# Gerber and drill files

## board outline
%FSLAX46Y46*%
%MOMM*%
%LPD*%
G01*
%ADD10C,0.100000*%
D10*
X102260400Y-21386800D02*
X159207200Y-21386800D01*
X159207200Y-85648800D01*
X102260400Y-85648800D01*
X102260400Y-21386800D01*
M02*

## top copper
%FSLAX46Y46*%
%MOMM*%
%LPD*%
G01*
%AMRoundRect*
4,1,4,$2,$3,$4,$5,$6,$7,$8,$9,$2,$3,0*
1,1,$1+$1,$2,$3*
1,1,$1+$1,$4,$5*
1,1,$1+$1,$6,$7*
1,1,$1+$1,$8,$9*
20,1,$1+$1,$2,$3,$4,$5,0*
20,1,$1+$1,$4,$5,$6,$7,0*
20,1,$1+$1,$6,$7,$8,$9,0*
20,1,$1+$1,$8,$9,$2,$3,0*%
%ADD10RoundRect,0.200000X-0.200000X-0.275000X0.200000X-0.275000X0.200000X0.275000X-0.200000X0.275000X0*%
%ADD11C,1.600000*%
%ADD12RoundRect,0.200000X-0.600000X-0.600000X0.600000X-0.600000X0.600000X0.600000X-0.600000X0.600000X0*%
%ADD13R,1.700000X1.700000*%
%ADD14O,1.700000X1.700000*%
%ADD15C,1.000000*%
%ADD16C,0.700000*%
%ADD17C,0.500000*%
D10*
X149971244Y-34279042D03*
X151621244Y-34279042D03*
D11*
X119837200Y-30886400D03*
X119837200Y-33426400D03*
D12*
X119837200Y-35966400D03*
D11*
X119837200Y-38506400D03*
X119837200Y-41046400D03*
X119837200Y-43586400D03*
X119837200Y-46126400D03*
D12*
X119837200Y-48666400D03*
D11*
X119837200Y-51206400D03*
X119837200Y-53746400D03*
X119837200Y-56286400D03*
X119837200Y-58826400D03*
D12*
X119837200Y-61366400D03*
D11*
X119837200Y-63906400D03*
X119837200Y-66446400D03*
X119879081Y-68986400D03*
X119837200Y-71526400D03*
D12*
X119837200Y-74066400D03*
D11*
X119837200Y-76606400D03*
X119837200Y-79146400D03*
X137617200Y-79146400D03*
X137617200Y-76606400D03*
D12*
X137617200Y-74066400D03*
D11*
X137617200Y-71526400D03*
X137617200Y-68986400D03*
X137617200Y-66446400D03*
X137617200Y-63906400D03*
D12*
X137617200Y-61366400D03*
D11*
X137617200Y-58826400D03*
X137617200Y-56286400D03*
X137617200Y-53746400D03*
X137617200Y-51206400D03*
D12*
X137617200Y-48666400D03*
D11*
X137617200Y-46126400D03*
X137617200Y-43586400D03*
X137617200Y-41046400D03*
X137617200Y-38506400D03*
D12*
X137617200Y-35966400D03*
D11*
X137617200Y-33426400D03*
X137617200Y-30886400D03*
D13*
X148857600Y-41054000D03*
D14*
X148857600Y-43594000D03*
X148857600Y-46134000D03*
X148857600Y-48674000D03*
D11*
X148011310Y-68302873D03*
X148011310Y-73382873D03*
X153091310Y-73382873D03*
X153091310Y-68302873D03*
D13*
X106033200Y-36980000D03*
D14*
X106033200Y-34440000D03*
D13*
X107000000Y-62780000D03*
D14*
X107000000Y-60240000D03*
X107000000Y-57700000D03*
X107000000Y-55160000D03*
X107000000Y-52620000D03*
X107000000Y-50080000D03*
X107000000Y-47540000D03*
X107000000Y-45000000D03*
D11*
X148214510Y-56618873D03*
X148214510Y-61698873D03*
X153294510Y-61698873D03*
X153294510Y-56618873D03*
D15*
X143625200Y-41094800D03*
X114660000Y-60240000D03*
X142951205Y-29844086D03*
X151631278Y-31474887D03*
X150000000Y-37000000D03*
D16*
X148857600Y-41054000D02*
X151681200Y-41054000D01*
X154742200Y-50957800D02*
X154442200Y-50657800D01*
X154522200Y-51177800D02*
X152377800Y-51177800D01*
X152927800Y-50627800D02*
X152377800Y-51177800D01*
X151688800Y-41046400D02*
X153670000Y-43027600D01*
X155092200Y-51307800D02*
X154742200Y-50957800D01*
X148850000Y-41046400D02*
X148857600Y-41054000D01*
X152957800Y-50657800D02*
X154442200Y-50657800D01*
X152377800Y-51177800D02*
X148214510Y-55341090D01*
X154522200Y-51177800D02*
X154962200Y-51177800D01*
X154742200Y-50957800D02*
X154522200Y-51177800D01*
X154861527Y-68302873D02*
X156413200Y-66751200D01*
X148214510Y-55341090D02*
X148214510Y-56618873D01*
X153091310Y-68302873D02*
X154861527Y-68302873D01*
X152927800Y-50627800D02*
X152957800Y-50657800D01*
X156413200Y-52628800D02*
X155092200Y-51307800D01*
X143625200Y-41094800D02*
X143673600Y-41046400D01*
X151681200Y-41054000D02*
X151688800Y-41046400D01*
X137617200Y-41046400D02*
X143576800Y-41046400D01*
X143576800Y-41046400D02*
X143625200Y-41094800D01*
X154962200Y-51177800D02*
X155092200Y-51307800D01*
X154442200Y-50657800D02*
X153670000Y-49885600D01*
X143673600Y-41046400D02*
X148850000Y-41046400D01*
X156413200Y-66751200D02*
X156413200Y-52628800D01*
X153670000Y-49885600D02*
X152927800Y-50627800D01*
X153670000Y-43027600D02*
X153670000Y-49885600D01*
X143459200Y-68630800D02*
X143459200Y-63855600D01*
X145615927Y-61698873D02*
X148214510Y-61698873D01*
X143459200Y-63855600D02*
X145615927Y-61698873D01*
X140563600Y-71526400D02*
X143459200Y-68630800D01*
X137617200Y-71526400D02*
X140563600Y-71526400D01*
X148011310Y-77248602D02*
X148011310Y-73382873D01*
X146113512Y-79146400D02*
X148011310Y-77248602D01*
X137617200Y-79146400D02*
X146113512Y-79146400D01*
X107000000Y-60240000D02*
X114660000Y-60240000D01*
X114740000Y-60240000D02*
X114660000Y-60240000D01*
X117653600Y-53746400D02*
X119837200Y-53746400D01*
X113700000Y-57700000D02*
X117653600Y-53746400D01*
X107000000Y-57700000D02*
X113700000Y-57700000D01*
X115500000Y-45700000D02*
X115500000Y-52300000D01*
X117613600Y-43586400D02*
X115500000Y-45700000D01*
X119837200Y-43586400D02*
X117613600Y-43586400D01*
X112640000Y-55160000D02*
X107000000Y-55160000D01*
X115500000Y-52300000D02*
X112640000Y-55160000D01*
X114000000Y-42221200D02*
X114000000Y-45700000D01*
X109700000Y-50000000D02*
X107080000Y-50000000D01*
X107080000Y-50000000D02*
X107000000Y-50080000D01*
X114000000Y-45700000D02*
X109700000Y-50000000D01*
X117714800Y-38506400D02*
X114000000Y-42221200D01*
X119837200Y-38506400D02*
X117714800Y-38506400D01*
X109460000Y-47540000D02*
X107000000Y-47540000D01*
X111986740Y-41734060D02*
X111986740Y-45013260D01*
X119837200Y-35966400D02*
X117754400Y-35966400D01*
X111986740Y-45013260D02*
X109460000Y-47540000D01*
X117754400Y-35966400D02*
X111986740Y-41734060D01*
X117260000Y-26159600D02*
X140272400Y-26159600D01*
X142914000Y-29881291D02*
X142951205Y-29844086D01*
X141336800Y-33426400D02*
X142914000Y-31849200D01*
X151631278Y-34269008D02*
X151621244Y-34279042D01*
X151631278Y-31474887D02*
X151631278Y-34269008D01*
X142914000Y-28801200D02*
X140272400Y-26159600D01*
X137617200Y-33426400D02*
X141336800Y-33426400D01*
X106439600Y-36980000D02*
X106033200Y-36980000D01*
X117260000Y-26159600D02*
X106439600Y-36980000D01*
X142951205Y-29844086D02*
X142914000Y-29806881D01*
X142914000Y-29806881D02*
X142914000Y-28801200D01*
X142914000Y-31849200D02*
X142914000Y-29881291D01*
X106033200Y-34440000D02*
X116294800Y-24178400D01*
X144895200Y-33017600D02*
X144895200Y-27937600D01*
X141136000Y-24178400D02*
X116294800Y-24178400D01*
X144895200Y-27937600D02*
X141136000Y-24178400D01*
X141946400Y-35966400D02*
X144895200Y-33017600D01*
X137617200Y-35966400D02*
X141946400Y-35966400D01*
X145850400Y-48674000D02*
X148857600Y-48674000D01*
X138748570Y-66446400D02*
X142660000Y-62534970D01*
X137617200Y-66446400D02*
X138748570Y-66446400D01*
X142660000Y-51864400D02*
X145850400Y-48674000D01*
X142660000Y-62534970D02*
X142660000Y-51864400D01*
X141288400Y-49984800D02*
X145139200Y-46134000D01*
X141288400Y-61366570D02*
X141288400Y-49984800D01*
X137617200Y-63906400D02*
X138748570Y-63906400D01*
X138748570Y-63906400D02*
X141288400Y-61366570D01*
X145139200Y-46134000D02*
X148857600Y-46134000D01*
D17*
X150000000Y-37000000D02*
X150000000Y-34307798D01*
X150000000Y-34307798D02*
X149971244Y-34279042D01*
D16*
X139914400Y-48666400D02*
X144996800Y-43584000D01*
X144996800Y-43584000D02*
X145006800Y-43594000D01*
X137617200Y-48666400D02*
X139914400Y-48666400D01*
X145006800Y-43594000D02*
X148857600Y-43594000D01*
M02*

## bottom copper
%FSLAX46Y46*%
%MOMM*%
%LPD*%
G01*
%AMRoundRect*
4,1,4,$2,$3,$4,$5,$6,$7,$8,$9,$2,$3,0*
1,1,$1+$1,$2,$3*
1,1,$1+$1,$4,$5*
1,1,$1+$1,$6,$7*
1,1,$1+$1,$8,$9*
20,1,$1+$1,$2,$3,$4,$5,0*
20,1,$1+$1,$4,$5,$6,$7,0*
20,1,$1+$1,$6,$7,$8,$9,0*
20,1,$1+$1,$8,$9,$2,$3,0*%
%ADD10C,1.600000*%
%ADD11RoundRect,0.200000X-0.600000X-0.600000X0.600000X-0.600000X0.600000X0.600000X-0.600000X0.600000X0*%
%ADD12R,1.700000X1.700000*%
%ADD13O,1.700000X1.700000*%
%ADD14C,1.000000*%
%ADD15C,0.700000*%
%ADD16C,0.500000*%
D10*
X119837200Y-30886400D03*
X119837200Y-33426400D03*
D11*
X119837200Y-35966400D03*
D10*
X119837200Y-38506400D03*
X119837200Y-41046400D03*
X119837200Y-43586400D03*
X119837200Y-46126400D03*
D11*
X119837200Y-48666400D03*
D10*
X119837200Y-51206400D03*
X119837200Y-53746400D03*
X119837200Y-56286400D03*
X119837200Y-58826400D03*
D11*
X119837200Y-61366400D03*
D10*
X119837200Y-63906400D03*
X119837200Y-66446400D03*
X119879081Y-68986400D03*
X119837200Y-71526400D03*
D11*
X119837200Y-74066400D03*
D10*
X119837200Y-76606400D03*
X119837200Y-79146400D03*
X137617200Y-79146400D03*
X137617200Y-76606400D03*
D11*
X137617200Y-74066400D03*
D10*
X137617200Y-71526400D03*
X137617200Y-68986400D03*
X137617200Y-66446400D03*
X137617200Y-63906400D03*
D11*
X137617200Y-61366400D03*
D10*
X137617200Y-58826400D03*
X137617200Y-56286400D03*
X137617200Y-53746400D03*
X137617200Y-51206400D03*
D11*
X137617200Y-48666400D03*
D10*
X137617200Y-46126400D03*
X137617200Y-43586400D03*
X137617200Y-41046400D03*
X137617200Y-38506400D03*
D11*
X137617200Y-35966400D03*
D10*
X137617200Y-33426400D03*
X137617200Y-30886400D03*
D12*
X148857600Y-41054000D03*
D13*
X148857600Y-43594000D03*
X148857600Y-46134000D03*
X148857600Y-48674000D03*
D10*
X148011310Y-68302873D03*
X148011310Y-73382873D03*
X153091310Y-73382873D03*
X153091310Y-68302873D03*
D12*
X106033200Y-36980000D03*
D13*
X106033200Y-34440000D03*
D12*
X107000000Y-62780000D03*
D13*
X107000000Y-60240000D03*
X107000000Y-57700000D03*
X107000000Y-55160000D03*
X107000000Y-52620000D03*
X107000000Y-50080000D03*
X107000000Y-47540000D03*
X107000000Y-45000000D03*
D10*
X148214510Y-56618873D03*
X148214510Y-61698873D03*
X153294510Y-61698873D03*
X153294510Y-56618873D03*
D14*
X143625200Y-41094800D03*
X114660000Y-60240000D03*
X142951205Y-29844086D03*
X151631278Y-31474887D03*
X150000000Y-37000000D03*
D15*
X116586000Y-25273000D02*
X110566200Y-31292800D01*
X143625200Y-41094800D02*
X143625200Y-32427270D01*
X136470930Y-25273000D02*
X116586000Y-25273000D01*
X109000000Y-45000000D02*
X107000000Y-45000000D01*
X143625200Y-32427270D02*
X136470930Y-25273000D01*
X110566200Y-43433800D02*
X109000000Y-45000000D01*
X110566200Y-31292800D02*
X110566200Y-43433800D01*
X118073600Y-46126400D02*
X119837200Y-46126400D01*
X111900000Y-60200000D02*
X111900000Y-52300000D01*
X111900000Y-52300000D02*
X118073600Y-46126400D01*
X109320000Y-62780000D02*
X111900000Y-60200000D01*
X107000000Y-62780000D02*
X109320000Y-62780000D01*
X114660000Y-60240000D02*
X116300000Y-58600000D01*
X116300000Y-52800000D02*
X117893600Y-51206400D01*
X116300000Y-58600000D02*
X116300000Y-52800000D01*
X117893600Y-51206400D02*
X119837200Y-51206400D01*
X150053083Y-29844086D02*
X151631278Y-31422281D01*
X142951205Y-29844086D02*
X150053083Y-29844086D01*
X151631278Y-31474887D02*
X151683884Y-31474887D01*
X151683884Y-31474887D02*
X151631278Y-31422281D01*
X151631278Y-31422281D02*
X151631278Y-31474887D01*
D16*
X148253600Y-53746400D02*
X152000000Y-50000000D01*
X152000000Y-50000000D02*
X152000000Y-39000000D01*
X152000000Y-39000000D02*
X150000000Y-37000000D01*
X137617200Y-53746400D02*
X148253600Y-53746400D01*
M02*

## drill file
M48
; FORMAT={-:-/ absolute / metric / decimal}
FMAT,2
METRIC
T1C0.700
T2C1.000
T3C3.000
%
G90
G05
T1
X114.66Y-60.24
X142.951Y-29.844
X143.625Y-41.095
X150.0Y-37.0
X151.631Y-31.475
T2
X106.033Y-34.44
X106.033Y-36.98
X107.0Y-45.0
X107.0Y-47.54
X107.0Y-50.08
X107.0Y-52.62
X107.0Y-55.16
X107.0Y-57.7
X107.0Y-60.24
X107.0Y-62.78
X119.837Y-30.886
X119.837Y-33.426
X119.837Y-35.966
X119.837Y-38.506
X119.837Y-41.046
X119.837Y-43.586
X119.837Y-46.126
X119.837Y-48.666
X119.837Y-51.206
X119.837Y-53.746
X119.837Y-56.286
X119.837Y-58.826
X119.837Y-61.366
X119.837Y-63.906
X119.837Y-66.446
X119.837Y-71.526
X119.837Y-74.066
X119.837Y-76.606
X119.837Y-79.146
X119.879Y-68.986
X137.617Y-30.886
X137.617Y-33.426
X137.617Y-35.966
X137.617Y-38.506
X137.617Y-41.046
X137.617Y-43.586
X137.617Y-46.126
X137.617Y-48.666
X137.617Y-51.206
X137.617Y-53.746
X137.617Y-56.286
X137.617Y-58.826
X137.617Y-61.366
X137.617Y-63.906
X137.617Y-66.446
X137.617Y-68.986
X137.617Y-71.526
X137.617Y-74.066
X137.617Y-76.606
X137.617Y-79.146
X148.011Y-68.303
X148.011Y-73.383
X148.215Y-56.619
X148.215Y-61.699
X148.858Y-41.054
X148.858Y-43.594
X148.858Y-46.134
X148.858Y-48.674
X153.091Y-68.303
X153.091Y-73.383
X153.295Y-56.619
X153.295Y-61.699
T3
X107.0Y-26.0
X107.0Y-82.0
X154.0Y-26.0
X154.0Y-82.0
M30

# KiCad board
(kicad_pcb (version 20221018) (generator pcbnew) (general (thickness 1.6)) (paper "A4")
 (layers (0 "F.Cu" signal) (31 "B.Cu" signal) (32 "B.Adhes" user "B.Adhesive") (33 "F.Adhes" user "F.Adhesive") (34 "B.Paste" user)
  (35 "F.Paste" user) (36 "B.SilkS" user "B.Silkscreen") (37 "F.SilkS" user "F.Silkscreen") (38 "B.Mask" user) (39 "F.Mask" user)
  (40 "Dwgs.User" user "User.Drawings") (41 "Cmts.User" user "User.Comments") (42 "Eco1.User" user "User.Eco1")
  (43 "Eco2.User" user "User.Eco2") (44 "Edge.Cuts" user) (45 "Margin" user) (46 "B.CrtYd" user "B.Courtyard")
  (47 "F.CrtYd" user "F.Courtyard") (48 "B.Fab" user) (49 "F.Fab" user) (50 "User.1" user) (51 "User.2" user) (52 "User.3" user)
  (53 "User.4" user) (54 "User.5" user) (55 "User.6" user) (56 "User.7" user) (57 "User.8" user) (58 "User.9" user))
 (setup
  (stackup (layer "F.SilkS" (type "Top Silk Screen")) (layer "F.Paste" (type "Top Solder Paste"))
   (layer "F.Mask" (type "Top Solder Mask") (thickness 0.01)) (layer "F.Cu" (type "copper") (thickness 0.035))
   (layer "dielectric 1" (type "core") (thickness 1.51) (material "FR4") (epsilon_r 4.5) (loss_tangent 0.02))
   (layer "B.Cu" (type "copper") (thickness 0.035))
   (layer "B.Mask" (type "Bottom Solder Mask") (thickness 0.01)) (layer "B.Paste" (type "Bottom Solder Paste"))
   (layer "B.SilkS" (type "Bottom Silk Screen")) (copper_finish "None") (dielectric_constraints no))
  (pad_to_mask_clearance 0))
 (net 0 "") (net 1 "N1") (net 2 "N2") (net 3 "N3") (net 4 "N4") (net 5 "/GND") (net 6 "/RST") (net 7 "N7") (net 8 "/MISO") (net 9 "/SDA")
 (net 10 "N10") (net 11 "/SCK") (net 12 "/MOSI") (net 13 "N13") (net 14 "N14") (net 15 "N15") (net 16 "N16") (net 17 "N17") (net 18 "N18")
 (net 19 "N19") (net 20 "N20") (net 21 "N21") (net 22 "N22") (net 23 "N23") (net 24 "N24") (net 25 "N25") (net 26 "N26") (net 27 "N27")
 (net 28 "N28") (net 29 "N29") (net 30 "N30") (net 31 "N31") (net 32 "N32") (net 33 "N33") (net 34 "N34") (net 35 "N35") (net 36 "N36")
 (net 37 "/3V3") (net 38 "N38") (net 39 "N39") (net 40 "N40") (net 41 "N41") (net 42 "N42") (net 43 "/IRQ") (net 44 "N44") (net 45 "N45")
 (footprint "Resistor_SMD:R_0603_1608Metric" (layer "F.Cu") (at 150.796244 34.279042)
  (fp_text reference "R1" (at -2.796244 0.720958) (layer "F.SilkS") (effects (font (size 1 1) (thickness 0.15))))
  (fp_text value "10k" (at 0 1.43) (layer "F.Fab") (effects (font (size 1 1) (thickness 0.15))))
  (pad "1" smd roundrect (at -0.825 0) (size 0.8 0.95) (layers "F.Cu" "F.Paste" "F.Mask") (roundrect_rratio 0.25) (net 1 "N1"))
  (pad "2" smd roundrect (at 0.825 0) (size 0.8 0.95) (layers "F.Cu" "F.Paste" "F.Mask") (roundrect_rratio 0.25) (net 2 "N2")))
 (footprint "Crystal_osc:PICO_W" (layer "F.Cu") (at 128.7272 55.0164)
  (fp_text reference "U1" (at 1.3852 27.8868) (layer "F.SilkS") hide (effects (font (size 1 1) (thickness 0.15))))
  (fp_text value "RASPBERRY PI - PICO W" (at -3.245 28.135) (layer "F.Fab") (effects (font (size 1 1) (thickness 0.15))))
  (pad "1" thru_hole circle (at -8.89 -24.13) (size 1.6 1.6) (drill 1) (layers "*.Cu" "*.Mask") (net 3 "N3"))
  (pad "2" thru_hole circle (at -8.89 -21.59) (size 1.6 1.6) (drill 1) (layers "*.Cu" "*.Mask") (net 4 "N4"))
  (pad "3" thru_hole roundrect (at -8.89 -19.05) (size 1.6 1.6) (drill 1) (layers "*.Cu" "*.Mask") (roundrect_rratio 0.125) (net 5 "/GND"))
  (pad "4" thru_hole circle (at -8.89 -16.51) (size 1.6 1.6) (drill 1) (layers "*.Cu" "*.Mask") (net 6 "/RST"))
  (pad "5" thru_hole circle (at -8.89 -13.97) (size 1.6 1.6) (drill 1) (layers "*.Cu" "*.Mask") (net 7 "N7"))
  (pad "6" thru_hole circle (at -8.89 -11.43) (size 1.6 1.6) (drill 1) (layers "*.Cu" "*.Mask") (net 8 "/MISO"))
  (pad "7" thru_hole circle (at -8.89 -8.89) (size 1.6 1.6) (drill 1) (layers "*.Cu" "*.Mask") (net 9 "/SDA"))
  (pad "8" thru_hole roundrect (at -8.89 -6.35) (size 1.6 1.6) (drill 1) (layers "*.Cu" "*.Mask") (roundrect_rratio 0.125) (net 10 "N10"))
  (pad "9" thru_hole circle (at -8.89 -3.81) (size 1.6 1.6) (drill 1) (layers "*.Cu" "*.Mask") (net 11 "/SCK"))
  (pad "10" thru_hole circle (at -8.89 -1.27) (size 1.6 1.6) (drill 1) (layers "*.Cu" "*.Mask") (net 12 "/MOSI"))
  (pad "11" thru_hole circle (at -8.89 1.27) (size 1.6 1.6) (drill 1) (layers "*.Cu" "*.Mask") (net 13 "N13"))
  (pad "12" thru_hole circle (at -8.89 3.81) (size 1.6 1.6) (drill 1) (layers "*.Cu" "*.Mask") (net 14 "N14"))
  (pad "13" thru_hole roundrect (at -8.89 6.35) (size 1.6 1.6) (drill 1) (layers "*.Cu" "*.Mask") (roundrect_rratio 0.125) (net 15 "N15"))
  (pad "14" thru_hole circle (at -8.89 8.89) (size 1.6 1.6) (drill 1) (layers "*.Cu" "*.Mask") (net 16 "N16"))
  (pad "15" thru_hole circle (at -8.89 11.43) (size 1.6 1.6) (drill 1) (layers "*.Cu" "*.Mask") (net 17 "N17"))
  (pad "16" thru_hole circle (at -8.848119 13.97) (size 1.6 1.6) (drill 1) (layers "*.Cu" "*.Mask") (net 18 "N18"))
  (pad "17" thru_hole circle (at -8.89 16.51) (size 1.6 1.6) (drill 1) (layers "*.Cu" "*.Mask") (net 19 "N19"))
  (pad "18" thru_hole roundrect (at -8.89 19.05) (size 1.6 1.6) (drill 1) (layers "*.Cu" "*.Mask") (roundrect_rratio 0.125) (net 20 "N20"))
  (pad "19" thru_hole circle (at -8.89 21.59) (size 1.6 1.6) (drill 1) (layers "*.Cu" "*.Mask") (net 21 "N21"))
  (pad "20" thru_hole circle (at -8.89 24.13) (size 1.6 1.6) (drill 1) (layers "*.Cu" "*.Mask") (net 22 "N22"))
  (pad "21" thru_hole circle (at 8.89 24.13) (size 1.6 1.6) (drill 1) (layers "*.Cu" "*.Mask") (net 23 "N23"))
  (pad "22" thru_hole circle (at 8.89 21.59) (size 1.6 1.6) (drill 1) (layers "*.Cu" "*.Mask") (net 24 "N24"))
  (pad "23" thru_hole roundrect (at 8.89 19.05) (size 1.6 1.6) (drill 1) (layers "*.Cu" "*.Mask") (roundrect_rratio 0.125) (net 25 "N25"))
  (pad "24" thru_hole circle (at 8.89 16.51) (size 1.6 1.6) (drill 1) (layers "*.Cu" "*.Mask") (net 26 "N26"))
  (pad "25" thru_hole circle (at 8.89 13.97) (size 1.6 1.6) (drill 1) (layers "*.Cu" "*.Mask") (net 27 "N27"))
  (pad "26" thru_hole circle (at 8.89 11.43) (size 1.6 1.6) (drill 1) (layers "*.Cu" "*.Mask") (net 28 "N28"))
  (pad "27" thru_hole circle (at 8.89 8.89) (size 1.6 1.6) (drill 1) (layers "*.Cu" "*.Mask") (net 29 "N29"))
  (pad "28" thru_hole roundrect (at 8.89 6.35) (size 1.6 1.6) (drill 1) (layers "*.Cu" "*.Mask") (roundrect_rratio 0.125) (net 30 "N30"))
  (pad "29" thru_hole circle (at 8.89 3.81) (size 1.6 1.6) (drill 1) (layers "*.Cu" "*.Mask") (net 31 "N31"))
  (pad "30" thru_hole circle (at 8.89 1.27) (size 1.6 1.6) (drill 1) (layers "*.Cu" "*.Mask") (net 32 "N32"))
  (pad "31" thru_hole circle (at 8.89 -1.27) (size 1.6 1.6) (drill 1) (layers "*.Cu" "*.Mask") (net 1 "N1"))
  (pad "32" thru_hole circle (at 8.89 -3.81) (size 1.6 1.6) (drill 1) (layers "*.Cu" "*.Mask") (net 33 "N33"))
  (pad "33" thru_hole roundrect (at 8.89 -6.35) (size 1.6 1.6) (drill 1) (layers "*.Cu" "*.Mask") (roundrect_rratio 0.125) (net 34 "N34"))
  (pad "34" thru_hole circle (at 8.89 -8.89) (size 1.6 1.6) (drill 1) (layers "*.Cu" "*.Mask") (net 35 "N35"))
  (pad "35" thru_hole circle (at 8.89 -11.43) (size 1.6 1.6) (drill 1) (layers "*.Cu" "*.Mask") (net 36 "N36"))
  (pad "36" thru_hole circle (at 8.89 -13.97) (size 1.6 1.6) (drill 1) (layers "*.Cu" "*.Mask") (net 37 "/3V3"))
  (pad "37" thru_hole circle (at 8.89 -16.51) (size 1.6 1.6) (drill 1) (layers "*.Cu" "*.Mask") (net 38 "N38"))
  (pad "38" thru_hole roundrect (at 8.89 -19.05) (size 1.6 1.6) (drill 1) (layers "*.Cu" "*.Mask") (roundrect_rratio 0.125) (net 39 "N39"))
  (pad "39" thru_hole circle (at 8.89 -21.59) (size 1.6 1.6) (drill 1) (layers "*.Cu" "*.Mask") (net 2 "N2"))
  (pad "40" thru_hole circle (at 8.89 -24.13) (size 1.6 1.6) (drill 1) (layers "*.Cu" "*.Mask") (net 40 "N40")))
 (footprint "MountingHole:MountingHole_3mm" (layer "F.Cu") (at 154 82)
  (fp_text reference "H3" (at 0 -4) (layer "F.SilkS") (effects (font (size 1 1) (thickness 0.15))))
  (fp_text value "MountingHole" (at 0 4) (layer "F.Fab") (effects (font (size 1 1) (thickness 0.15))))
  (pad "" np_thru_hole circle (at 0 0) (size 3 3) (drill 3) (layers "*.Cu" "*.Mask")))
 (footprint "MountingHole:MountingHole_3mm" (layer "F.Cu") (at 154 26)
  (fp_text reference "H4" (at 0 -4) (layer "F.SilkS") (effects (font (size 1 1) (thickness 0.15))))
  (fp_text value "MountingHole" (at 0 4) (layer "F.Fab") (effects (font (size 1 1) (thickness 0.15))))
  (pad "" np_thru_hole circle (at 0 0) (size 3 3) (drill 3) (layers "*.Cu" "*.Mask")))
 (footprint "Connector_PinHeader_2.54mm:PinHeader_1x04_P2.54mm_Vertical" (layer "F.Cu") (at 148.8576 41.054)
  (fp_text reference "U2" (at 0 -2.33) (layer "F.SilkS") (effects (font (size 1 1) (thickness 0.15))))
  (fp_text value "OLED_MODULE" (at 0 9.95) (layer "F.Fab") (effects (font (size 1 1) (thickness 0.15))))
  (pad "1" thru_hole rect (at 0 0) (size 1.7 1.7) (drill 1) (layers "*.Cu" "*.Mask") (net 37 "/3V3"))
  (pad "2" thru_hole oval (at 0 2.54) (size 1.7 1.7) (drill 1) (layers "*.Cu" "*.Mask") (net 34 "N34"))
  (pad "3" thru_hole oval (at 0 5.08) (size 1.7 1.7) (drill 1) (layers "*.Cu" "*.Mask") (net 29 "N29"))
  (pad "4" thru_hole oval (at 0 7.62) (size 1.7 1.7) (drill 1) (layers "*.Cu" "*.Mask") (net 28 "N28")))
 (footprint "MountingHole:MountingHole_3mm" (layer "F.Cu") (at 107 82)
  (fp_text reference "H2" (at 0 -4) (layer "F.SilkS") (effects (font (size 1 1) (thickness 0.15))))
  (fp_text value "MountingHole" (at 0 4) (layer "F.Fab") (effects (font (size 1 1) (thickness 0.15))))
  (pad "" np_thru_hole circle (at 0 0) (size 3 3) (drill 3) (layers "*.Cu" "*.Mask")))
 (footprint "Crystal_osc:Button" (layer "F.Cu") (at 150.55131 60.682873)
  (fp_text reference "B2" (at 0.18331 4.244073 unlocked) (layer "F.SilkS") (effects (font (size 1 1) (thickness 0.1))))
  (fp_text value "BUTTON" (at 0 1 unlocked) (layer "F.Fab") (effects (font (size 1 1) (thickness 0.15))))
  (pad "1" thru_hole circle (at -2.54 7.62) (size 1.6 1.6) (drill 1) (layers "*.Cu" "*.Mask") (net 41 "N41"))
  (pad "2" thru_hole circle (at -2.54 12.7) (size 1.6 1.6) (drill 1) (layers "*.Cu" "*.Mask") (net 23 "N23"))
  (pad "3" thru_hole circle (at 2.54 12.7 180) (size 1.6 1.6) (drill 1) (layers "*.Cu" "*.Mask") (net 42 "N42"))
  (pad "4" thru_hole circle (at 2.54 7.62 90) (size 1.6 1.6) (drill 1) (layers "*.Cu" "*.Mask") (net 37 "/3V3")))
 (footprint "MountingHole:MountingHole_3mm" (layer "F.Cu") (at 107 26)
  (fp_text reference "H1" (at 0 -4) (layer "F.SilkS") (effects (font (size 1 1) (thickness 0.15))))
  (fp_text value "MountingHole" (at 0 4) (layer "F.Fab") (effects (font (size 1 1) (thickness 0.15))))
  (pad "" np_thru_hole circle (at 0 0) (size 3 3) (drill 3) (layers "*.Cu" "*.Mask")))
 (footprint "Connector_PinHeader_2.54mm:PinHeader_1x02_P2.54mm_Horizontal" (layer "F.Cu") (at 106.0332 36.98 180)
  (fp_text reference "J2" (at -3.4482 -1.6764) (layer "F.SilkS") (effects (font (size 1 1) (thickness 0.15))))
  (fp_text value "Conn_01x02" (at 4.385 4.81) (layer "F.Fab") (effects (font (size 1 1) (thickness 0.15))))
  (pad "1" thru_hole rect (at 0 0 180) (size 1.7 1.7) (drill 1) (layers "*.Cu" "*.Mask") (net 2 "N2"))
  (pad "2" thru_hole oval (at 0 2.54 180) (size 1.7 1.7) (drill 1) (layers "*.Cu" "*.Mask") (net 39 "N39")))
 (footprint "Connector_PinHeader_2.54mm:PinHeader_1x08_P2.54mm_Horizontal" (layer "F.Cu") (at 107 62.78 180)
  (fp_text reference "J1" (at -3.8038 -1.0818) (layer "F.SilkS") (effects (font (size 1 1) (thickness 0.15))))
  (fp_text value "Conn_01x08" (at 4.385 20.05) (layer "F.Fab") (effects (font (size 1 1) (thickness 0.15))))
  (pad "1" thru_hole rect (at 0 0 180) (size 1.7 1.7) (drill 1) (layers "*.Cu" "*.Mask") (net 9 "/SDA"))
  (pad "2" thru_hole oval (at 0 2.54 180) (size 1.7 1.7) (drill 1) (layers "*.Cu" "*.Mask") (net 11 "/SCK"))
  (pad "3" thru_hole oval (at 0 5.08 180) (size 1.7 1.7) (drill 1) (layers "*.Cu" "*.Mask") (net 12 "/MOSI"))
  (pad "4" thru_hole oval (at 0 7.62 180) (size 1.7 1.7) (drill 1) (layers "*.Cu" "*.Mask") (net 8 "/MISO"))
  (pad "5" thru_hole oval (at 0 10.16 180) (size 1.7 1.7) (drill 1) (layers "*.Cu" "*.Mask") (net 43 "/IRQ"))
  (pad "6" thru_hole oval (at 0 12.7 180) (size 1.7 1.7) (drill 1) (layers "*.Cu" "*.Mask") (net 6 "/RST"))
  (pad "7" thru_hole oval (at 0 15.24 180) (size 1.7 1.7) (drill 1) (layers "*.Cu" "*.Mask") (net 5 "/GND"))
  (pad "8" thru_hole oval (at 0 17.78 180) (size 1.7 1.7) (drill 1) (layers "*.Cu" "*.Mask") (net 37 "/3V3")))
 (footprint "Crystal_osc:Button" (layer "F.Cu") (at 150.75451 48.998873)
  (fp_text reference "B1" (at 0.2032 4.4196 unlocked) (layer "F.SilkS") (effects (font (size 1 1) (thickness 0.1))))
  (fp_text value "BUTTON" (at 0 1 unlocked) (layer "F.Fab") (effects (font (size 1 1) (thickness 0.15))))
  (pad "1" thru_hole circle (at -2.54 7.62) (size 1.6 1.6) (drill 1) (layers "*.Cu" "*.Mask") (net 37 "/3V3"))
  (pad "2" thru_hole circle (at -2.54 12.7) (size 1.6 1.6) (drill 1) (layers "*.Cu" "*.Mask") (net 26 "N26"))
  (pad "3" thru_hole circle (at 2.54 12.7 180) (size 1.6 1.6) (drill 1) (layers "*.Cu" "*.Mask") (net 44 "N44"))
  (pad "4" thru_hole circle (at 2.54 7.62 90) (size 1.6 1.6) (drill 1) (layers "*.Cu" "*.Mask") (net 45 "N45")))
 (gr_rect (start 102.2604 21.3868) (end 159.2072 85.6488) (stroke (width 0.1) (type default)) (fill none) (layer "Edge.Cuts"))
 (segment (start 148.8576 41.054) (end 151.6812 41.054) (width 0.7) (layer "F.Cu") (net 37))
 (segment (start 154.7422 50.9578) (end 154.4422 50.6578) (width 0.7) (layer "F.Cu") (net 37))
 (segment (start 154.5222 51.1778) (end 152.3778 51.1778) (width 0.7) (layer "F.Cu") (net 37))
 (segment (start 152.9278 50.6278) (end 152.3778 51.1778) (width 0.7) (layer "F.Cu") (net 37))
 (segment (start 151.6888 41.0464) (end 153.67 43.0276) (width 0.7) (layer "F.Cu") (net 37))
 (segment (start 155.0922 51.3078) (end 154.7422 50.9578) (width 0.7) (layer "F.Cu") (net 37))
 (segment (start 148.85 41.0464) (end 148.8576 41.054) (width 0.7) (layer "F.Cu") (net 37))
 (segment (start 152.9578 50.6578) (end 154.4422 50.6578) (width 0.7) (layer "F.Cu") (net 37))
 (segment (start 152.3778 51.1778) (end 148.21451 55.34109) (width 0.7) (layer "F.Cu") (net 37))
 (segment (start 154.5222 51.1778) (end 154.9622 51.1778) (width 0.7) (layer "F.Cu") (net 37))
 (segment (start 154.7422 50.9578) (end 154.5222 51.1778) (width 0.7) (layer "F.Cu") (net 37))
 (segment (start 154.861527 68.302873) (end 156.4132 66.7512) (width 0.7) (layer "F.Cu") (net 37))
 (segment (start 148.21451 55.34109) (end 148.21451 56.618873) (width 0.7) (layer "F.Cu") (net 37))
 (segment (start 153.09131 68.302873) (end 154.861527 68.302873) (width 0.7) (layer "F.Cu") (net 37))
 (segment (start 152.9278 50.6278) (end 152.9578 50.6578) (width 0.7) (layer "F.Cu") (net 37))
 (segment (start 156.4132 52.6288) (end 155.0922 51.3078) (width 0.7) (layer "F.Cu") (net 37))
 (segment (start 143.6252 41.0948) (end 143.6736 41.0464) (width 0.7) (layer "F.Cu") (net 37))
 (segment (start 151.6812 41.054) (end 151.6888 41.0464) (width 0.7) (layer "F.Cu") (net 37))
 (segment (start 137.6172 41.0464) (end 143.5768 41.0464) (width 0.7) (layer "F.Cu") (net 37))
 (segment (start 143.5768 41.0464) (end 143.6252 41.0948) (width 0.7) (layer "F.Cu") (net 37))
 (segment (start 154.9622 51.1778) (end 155.0922 51.3078) (width 0.7) (layer "F.Cu") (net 37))
 (segment (start 154.4422 50.6578) (end 153.67 49.8856) (width 0.7) (layer "F.Cu") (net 37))
 (segment (start 143.6736 41.0464) (end 148.85 41.0464) (width 0.7) (layer "F.Cu") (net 37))
 (segment (start 156.4132 66.7512) (end 156.4132 52.6288) (width 0.7) (layer "F.Cu") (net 37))
 (segment (start 153.67 49.8856) (end 152.9278 50.6278) (width 0.7) (layer "F.Cu") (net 37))
 (segment (start 153.67 43.0276) (end 153.67 49.8856) (width 0.7) (layer "F.Cu") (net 37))
 (via (at 143.6252 41.0948) (size 1) (drill 0.7) (layers "F.Cu" "B.Cu") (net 37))
 (segment (start 116.586 25.273) (end 110.5662 31.2928) (width 0.7) (layer "B.Cu") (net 37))
 (segment (start 143.6252 41.0948) (end 143.6252 32.42727) (width 0.7) (layer "B.Cu") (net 37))
 (segment (start 136.47093 25.273) (end 116.586 25.273) (width 0.7) (layer "B.Cu") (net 37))
 (segment (start 109 45) (end 107 45) (width 0.7) (layer "B.Cu") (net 37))
 (segment (start 143.6252 32.42727) (end 136.47093 25.273) (width 0.7) (layer "B.Cu") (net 37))
 (segment (start 110.5662 43.4338) (end 109 45) (width 0.7) (layer "B.Cu") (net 37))
 (segment (start 110.5662 31.2928) (end 110.5662 43.4338) (width 0.7) (layer "B.Cu") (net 37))
 (segment (start 143.4592 68.6308) (end 143.4592 63.8556) (width 0.7) (layer "F.Cu") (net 26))
 (segment (start 145.615927 61.698873) (end 148.21451 61.698873) (width 0.7) (layer "F.Cu") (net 26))
 (segment (start 143.4592 63.8556) (end 145.615927 61.698873) (width 0.7) (layer "F.Cu") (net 26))
 (segment (start 140.5636 71.5264) (end 143.4592 68.6308) (width 0.7) (layer "F.Cu") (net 26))
 (segment (start 137.6172 71.5264) (end 140.5636 71.5264) (width 0.7) (layer "F.Cu") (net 26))
 (segment (start 148.01131 77.248602) (end 148.01131 73.382873) (width 0.7) (layer "F.Cu") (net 23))
 (segment (start 146.113512 79.1464) (end 148.01131 77.248602) (width 0.7) (layer "F.Cu") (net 23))
 (segment (start 137.6172 79.1464) (end 146.113512 79.1464) (width 0.7) (layer "F.Cu") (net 23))
 (segment (start 118.0736 46.1264) (end 119.8372 46.1264) (width 0.7) (layer "B.Cu") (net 9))
 (segment (start 111.9 60.2) (end 111.9 52.3) (width 0.7) (layer "B.Cu") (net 9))
 (segment (start 111.9 52.3) (end 118.0736 46.1264) (width 0.7) (layer "B.Cu") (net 9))
 (segment (start 109.32 62.78) (end 111.9 60.2) (width 0.7) (layer "B.Cu") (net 9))
 (segment (start 107 62.78) (end 109.32 62.78) (width 0.7) (layer "B.Cu") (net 9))
 (segment (start 107 60.24) (end 114.66 60.24) (width 0.7) (layer "F.Cu") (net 11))
 (segment (start 114.74 60.24) (end 114.66 60.24) (width 0.7) (layer "F.Cu") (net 11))
 (via (at 114.66 60.24) (size 1) (drill 0.7) (layers "F.Cu" "B.Cu") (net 11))
 (segment (start 114.66 60.24) (end 116.3 58.6) (width 0.7) (layer "B.Cu") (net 11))
 (segment (start 116.3 52.8) (end 117.8936 51.2064) (width 0.7) (layer "B.Cu") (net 11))
 (segment (start 116.3 58.6) (end 116.3 52.8) (width 0.7) (layer "B.Cu") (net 11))
 (segment (start 117.8936 51.2064) (end 119.8372 51.2064) (width 0.7) (layer "B.Cu") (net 11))
 (segment (start 117.6536 53.7464) (end 119.8372 53.7464) (width 0.7) (layer "F.Cu") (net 12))
 (segment (start 113.7 57.7) (end 117.6536 53.7464) (width 0.7) (layer "F.Cu") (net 12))
 (segment (start 107 57.7) (end 113.7 57.7) (width 0.7) (layer "F.Cu") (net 12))
 (segment (start 115.5 45.7) (end 115.5 52.3) (width 0.7) (layer "F.Cu") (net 8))
 (segment (start 117.6136 43.5864) (end 115.5 45.7) (width 0.7) (layer "F.Cu") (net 8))
 (segment (start 119.8372 43.5864) (end 117.6136 43.5864) (width 0.7) (layer "F.Cu") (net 8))
 (segment (start 112.64 55.16) (end 107 55.16) (width 0.7) (layer "F.Cu") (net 8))
 (segment (start 115.5 52.3) (end 112.64 55.16) (width 0.7) (layer "F.Cu") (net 8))
 (segment (start 114 42.2212) (end 114 45.7) (width 0.7) (layer "F.Cu") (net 6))
 (segment (start 109.7 50) (end 107.08 50) (width 0.7) (layer "F.Cu") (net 6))
 (segment (start 107.08 50) (end 107 50.08) (width 0.7) (layer "F.Cu") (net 6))
 (segment (start 114 45.7) (end 109.7 50) (width 0.7) (layer "F.Cu") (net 6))
 (segment (start 117.7148 38.5064) (end 114 42.2212) (width 0.7) (layer "F.Cu") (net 6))
 (segment (start 119.8372 38.5064) (end 117.7148 38.5064) (width 0.7) (layer "F.Cu") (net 6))
 (segment (start 109.46 47.54) (end 107 47.54) (width 0.7) (layer "F.Cu") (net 5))
 (segment (start 111.98674 41.73406) (end 111.98674 45.01326) (width 0.7) (layer "F.Cu") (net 5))
 (segment (start 119.8372 35.9664) (end 117.7544 35.9664) (width 0.7) (layer "F.Cu") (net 5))
 (segment (start 111.98674 45.01326) (end 109.46 47.54) (width 0.7) (layer "F.Cu") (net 5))
 (segment (start 117.7544 35.9664) (end 111.98674 41.73406) (width 0.7) (layer "F.Cu") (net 5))
 (segment (start 117.26 26.1596) (end 140.2724 26.1596) (width 0.7) (layer "F.Cu") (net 2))
 (segment (start 142.914 29.881291) (end 142.951205 29.844086) (width 0.7) (layer "F.Cu") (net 2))
 (segment (start 141.3368 33.4264) (end 142.914 31.8492) (width 0.7) (layer "F.Cu") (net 2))
 (segment (start 151.631278 34.269008) (end 151.621244 34.279042) (width 0.7) (layer "F.Cu") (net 2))
 (segment (start 151.631278 31.474887) (end 151.631278 34.269008) (width 0.7) (layer "F.Cu") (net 2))
 (segment (start 142.914 28.8012) (end 140.2724 26.1596) (width 0.7) (layer "F.Cu") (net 2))
 (segment (start 137.6172 33.4264) (end 141.3368 33.4264) (width 0.7) (layer "F.Cu") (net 2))
 (segment (start 106.4396 36.98) (end 106.0332 36.98) (width 0.7) (layer "F.Cu") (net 2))
 (segment (start 117.26 26.1596) (end 106.4396 36.98) (width 0.7) (layer "F.Cu") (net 2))
 (segment (start 142.951205 29.844086) (end 142.914 29.806881) (width 0.7) (layer "F.Cu") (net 2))
 (segment (start 142.914 29.806881) (end 142.914 28.8012) (width 0.7) (layer "F.Cu") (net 2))
 (segment (start 142.914 31.8492) (end 142.914 29.881291) (width 0.7) (layer "F.Cu") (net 2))
 (via (at 142.951205 29.844086) (size 1) (drill 0.7) (layers "F.Cu" "B.Cu") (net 2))
 (via (at 151.631278 31.474887) (size 1) (drill 0.7) (layers "F.Cu" "B.Cu") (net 2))
 (segment (start 150.053083 29.844086) (end 151.631278 31.422281) (width 0.7) (layer "B.Cu") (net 2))
 (segment (start 142.951205 29.844086) (end 150.053083 29.844086) (width 0.7) (layer "B.Cu") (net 2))
 (segment (start 151.631278 31.474887) (end 151.683884 31.474887) (width 0.7) (layer "B.Cu") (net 2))
 (segment (start 151.683884 31.474887) (end 151.631278 31.422281) (width 0.7) (layer "B.Cu") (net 2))
 (segment (start 151.631278 31.422281) (end 151.631278 31.474887) (width 0.7) (layer "B.Cu") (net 2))
 (segment (start 106.0332 34.44) (end 116.2948 24.1784) (width 0.7) (layer "F.Cu") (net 39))
 (segment (start 144.8952 33.0176) (end 144.8952 27.9376) (width 0.7) (layer "F.Cu") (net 39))
 (segment (start 141.136 24.1784) (end 116.2948 24.1784) (width 0.7) (layer "F.Cu") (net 39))
 (segment (start 144.8952 27.9376) (end 141.136 24.1784) (width 0.7) (layer "F.Cu") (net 39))
 (segment (start 141.9464 35.9664) (end 144.8952 33.0176) (width 0.7) (layer "F.Cu") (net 39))
 (segment (start 137.6172 35.9664) (end 141.9464 35.9664) (width 0.7) (layer "F.Cu") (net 39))
 (segment (start 145.8504 48.674) (end 148.8576 48.674) (width 0.7) (layer "F.Cu") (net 28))
 (segment (start 138.74857 66.4464) (end 142.66 62.53497) (width 0.7) (layer "F.Cu") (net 28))
 (segment (start 137.6172 66.4464) (end 138.74857 66.4464) (width 0.7) (layer "F.Cu") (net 28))
 (segment (start 142.66 51.8644) (end 145.8504 48.674) (width 0.7) (layer "F.Cu") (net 28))
 (segment (start 142.66 62.53497) (end 142.66 51.8644) (width 0.7) (layer "F.Cu") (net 28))
 (segment (start 141.2884 49.9848) (end 145.1392 46.134) (width 0.7) (layer "F.Cu") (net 29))
 (segment (start 141.2884 61.36657) (end 141.2884 49.9848) (width 0.7) (layer "F.Cu") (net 29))
 (segment (start 137.6172 63.9064) (end 138.74857 63.9064) (width 0.7) (layer "F.Cu") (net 29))
 (segment (start 138.74857 63.9064) (end 141.2884 61.36657) (width 0.7) (layer "F.Cu") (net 29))
 (segment (start 145.1392 46.134) (end 148.8576 46.134) (width 0.7) (layer "F.Cu") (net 29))
 (segment (start 150 37) (end 150 34.307798) (width 0.5) (layer "F.Cu") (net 1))
 (segment (start 150 34.307798) (end 149.971244 34.279042) (width 0.5) (layer "F.Cu") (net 1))
 (via (at 150 37) (size 1) (drill 0.7) (layers "F.Cu" "B.Cu") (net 1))
 (segment (start 148.2536 53.7464) (end 152 50) (width 0.5) (layer "B.Cu") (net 1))
 (segment (start 152 50) (end 152 39) (width 0.5) (layer "B.Cu") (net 1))
 (segment (start 152 39) (end 150 37) (width 0.5) (layer "B.Cu") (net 1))
 (segment (start 137.6172 53.7464) (end 148.2536 53.7464) (width 0.5) (layer "B.Cu") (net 1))
 (segment (start 139.9144 48.6664) (end 144.9968 43.584) (width 0.7) (layer "F.Cu") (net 34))
 (segment (start 144.9968 43.584) (end 145.0068 43.594) (width 0.7) (layer "F.Cu") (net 34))
 (segment (start 137.6172 48.6664) (end 139.9144 48.6664) (width 0.7) (layer "F.Cu") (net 34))
 (segment (start 145.0068 43.594) (end 148.8576 43.594) (width 0.7) (layer "F.Cu") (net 34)))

